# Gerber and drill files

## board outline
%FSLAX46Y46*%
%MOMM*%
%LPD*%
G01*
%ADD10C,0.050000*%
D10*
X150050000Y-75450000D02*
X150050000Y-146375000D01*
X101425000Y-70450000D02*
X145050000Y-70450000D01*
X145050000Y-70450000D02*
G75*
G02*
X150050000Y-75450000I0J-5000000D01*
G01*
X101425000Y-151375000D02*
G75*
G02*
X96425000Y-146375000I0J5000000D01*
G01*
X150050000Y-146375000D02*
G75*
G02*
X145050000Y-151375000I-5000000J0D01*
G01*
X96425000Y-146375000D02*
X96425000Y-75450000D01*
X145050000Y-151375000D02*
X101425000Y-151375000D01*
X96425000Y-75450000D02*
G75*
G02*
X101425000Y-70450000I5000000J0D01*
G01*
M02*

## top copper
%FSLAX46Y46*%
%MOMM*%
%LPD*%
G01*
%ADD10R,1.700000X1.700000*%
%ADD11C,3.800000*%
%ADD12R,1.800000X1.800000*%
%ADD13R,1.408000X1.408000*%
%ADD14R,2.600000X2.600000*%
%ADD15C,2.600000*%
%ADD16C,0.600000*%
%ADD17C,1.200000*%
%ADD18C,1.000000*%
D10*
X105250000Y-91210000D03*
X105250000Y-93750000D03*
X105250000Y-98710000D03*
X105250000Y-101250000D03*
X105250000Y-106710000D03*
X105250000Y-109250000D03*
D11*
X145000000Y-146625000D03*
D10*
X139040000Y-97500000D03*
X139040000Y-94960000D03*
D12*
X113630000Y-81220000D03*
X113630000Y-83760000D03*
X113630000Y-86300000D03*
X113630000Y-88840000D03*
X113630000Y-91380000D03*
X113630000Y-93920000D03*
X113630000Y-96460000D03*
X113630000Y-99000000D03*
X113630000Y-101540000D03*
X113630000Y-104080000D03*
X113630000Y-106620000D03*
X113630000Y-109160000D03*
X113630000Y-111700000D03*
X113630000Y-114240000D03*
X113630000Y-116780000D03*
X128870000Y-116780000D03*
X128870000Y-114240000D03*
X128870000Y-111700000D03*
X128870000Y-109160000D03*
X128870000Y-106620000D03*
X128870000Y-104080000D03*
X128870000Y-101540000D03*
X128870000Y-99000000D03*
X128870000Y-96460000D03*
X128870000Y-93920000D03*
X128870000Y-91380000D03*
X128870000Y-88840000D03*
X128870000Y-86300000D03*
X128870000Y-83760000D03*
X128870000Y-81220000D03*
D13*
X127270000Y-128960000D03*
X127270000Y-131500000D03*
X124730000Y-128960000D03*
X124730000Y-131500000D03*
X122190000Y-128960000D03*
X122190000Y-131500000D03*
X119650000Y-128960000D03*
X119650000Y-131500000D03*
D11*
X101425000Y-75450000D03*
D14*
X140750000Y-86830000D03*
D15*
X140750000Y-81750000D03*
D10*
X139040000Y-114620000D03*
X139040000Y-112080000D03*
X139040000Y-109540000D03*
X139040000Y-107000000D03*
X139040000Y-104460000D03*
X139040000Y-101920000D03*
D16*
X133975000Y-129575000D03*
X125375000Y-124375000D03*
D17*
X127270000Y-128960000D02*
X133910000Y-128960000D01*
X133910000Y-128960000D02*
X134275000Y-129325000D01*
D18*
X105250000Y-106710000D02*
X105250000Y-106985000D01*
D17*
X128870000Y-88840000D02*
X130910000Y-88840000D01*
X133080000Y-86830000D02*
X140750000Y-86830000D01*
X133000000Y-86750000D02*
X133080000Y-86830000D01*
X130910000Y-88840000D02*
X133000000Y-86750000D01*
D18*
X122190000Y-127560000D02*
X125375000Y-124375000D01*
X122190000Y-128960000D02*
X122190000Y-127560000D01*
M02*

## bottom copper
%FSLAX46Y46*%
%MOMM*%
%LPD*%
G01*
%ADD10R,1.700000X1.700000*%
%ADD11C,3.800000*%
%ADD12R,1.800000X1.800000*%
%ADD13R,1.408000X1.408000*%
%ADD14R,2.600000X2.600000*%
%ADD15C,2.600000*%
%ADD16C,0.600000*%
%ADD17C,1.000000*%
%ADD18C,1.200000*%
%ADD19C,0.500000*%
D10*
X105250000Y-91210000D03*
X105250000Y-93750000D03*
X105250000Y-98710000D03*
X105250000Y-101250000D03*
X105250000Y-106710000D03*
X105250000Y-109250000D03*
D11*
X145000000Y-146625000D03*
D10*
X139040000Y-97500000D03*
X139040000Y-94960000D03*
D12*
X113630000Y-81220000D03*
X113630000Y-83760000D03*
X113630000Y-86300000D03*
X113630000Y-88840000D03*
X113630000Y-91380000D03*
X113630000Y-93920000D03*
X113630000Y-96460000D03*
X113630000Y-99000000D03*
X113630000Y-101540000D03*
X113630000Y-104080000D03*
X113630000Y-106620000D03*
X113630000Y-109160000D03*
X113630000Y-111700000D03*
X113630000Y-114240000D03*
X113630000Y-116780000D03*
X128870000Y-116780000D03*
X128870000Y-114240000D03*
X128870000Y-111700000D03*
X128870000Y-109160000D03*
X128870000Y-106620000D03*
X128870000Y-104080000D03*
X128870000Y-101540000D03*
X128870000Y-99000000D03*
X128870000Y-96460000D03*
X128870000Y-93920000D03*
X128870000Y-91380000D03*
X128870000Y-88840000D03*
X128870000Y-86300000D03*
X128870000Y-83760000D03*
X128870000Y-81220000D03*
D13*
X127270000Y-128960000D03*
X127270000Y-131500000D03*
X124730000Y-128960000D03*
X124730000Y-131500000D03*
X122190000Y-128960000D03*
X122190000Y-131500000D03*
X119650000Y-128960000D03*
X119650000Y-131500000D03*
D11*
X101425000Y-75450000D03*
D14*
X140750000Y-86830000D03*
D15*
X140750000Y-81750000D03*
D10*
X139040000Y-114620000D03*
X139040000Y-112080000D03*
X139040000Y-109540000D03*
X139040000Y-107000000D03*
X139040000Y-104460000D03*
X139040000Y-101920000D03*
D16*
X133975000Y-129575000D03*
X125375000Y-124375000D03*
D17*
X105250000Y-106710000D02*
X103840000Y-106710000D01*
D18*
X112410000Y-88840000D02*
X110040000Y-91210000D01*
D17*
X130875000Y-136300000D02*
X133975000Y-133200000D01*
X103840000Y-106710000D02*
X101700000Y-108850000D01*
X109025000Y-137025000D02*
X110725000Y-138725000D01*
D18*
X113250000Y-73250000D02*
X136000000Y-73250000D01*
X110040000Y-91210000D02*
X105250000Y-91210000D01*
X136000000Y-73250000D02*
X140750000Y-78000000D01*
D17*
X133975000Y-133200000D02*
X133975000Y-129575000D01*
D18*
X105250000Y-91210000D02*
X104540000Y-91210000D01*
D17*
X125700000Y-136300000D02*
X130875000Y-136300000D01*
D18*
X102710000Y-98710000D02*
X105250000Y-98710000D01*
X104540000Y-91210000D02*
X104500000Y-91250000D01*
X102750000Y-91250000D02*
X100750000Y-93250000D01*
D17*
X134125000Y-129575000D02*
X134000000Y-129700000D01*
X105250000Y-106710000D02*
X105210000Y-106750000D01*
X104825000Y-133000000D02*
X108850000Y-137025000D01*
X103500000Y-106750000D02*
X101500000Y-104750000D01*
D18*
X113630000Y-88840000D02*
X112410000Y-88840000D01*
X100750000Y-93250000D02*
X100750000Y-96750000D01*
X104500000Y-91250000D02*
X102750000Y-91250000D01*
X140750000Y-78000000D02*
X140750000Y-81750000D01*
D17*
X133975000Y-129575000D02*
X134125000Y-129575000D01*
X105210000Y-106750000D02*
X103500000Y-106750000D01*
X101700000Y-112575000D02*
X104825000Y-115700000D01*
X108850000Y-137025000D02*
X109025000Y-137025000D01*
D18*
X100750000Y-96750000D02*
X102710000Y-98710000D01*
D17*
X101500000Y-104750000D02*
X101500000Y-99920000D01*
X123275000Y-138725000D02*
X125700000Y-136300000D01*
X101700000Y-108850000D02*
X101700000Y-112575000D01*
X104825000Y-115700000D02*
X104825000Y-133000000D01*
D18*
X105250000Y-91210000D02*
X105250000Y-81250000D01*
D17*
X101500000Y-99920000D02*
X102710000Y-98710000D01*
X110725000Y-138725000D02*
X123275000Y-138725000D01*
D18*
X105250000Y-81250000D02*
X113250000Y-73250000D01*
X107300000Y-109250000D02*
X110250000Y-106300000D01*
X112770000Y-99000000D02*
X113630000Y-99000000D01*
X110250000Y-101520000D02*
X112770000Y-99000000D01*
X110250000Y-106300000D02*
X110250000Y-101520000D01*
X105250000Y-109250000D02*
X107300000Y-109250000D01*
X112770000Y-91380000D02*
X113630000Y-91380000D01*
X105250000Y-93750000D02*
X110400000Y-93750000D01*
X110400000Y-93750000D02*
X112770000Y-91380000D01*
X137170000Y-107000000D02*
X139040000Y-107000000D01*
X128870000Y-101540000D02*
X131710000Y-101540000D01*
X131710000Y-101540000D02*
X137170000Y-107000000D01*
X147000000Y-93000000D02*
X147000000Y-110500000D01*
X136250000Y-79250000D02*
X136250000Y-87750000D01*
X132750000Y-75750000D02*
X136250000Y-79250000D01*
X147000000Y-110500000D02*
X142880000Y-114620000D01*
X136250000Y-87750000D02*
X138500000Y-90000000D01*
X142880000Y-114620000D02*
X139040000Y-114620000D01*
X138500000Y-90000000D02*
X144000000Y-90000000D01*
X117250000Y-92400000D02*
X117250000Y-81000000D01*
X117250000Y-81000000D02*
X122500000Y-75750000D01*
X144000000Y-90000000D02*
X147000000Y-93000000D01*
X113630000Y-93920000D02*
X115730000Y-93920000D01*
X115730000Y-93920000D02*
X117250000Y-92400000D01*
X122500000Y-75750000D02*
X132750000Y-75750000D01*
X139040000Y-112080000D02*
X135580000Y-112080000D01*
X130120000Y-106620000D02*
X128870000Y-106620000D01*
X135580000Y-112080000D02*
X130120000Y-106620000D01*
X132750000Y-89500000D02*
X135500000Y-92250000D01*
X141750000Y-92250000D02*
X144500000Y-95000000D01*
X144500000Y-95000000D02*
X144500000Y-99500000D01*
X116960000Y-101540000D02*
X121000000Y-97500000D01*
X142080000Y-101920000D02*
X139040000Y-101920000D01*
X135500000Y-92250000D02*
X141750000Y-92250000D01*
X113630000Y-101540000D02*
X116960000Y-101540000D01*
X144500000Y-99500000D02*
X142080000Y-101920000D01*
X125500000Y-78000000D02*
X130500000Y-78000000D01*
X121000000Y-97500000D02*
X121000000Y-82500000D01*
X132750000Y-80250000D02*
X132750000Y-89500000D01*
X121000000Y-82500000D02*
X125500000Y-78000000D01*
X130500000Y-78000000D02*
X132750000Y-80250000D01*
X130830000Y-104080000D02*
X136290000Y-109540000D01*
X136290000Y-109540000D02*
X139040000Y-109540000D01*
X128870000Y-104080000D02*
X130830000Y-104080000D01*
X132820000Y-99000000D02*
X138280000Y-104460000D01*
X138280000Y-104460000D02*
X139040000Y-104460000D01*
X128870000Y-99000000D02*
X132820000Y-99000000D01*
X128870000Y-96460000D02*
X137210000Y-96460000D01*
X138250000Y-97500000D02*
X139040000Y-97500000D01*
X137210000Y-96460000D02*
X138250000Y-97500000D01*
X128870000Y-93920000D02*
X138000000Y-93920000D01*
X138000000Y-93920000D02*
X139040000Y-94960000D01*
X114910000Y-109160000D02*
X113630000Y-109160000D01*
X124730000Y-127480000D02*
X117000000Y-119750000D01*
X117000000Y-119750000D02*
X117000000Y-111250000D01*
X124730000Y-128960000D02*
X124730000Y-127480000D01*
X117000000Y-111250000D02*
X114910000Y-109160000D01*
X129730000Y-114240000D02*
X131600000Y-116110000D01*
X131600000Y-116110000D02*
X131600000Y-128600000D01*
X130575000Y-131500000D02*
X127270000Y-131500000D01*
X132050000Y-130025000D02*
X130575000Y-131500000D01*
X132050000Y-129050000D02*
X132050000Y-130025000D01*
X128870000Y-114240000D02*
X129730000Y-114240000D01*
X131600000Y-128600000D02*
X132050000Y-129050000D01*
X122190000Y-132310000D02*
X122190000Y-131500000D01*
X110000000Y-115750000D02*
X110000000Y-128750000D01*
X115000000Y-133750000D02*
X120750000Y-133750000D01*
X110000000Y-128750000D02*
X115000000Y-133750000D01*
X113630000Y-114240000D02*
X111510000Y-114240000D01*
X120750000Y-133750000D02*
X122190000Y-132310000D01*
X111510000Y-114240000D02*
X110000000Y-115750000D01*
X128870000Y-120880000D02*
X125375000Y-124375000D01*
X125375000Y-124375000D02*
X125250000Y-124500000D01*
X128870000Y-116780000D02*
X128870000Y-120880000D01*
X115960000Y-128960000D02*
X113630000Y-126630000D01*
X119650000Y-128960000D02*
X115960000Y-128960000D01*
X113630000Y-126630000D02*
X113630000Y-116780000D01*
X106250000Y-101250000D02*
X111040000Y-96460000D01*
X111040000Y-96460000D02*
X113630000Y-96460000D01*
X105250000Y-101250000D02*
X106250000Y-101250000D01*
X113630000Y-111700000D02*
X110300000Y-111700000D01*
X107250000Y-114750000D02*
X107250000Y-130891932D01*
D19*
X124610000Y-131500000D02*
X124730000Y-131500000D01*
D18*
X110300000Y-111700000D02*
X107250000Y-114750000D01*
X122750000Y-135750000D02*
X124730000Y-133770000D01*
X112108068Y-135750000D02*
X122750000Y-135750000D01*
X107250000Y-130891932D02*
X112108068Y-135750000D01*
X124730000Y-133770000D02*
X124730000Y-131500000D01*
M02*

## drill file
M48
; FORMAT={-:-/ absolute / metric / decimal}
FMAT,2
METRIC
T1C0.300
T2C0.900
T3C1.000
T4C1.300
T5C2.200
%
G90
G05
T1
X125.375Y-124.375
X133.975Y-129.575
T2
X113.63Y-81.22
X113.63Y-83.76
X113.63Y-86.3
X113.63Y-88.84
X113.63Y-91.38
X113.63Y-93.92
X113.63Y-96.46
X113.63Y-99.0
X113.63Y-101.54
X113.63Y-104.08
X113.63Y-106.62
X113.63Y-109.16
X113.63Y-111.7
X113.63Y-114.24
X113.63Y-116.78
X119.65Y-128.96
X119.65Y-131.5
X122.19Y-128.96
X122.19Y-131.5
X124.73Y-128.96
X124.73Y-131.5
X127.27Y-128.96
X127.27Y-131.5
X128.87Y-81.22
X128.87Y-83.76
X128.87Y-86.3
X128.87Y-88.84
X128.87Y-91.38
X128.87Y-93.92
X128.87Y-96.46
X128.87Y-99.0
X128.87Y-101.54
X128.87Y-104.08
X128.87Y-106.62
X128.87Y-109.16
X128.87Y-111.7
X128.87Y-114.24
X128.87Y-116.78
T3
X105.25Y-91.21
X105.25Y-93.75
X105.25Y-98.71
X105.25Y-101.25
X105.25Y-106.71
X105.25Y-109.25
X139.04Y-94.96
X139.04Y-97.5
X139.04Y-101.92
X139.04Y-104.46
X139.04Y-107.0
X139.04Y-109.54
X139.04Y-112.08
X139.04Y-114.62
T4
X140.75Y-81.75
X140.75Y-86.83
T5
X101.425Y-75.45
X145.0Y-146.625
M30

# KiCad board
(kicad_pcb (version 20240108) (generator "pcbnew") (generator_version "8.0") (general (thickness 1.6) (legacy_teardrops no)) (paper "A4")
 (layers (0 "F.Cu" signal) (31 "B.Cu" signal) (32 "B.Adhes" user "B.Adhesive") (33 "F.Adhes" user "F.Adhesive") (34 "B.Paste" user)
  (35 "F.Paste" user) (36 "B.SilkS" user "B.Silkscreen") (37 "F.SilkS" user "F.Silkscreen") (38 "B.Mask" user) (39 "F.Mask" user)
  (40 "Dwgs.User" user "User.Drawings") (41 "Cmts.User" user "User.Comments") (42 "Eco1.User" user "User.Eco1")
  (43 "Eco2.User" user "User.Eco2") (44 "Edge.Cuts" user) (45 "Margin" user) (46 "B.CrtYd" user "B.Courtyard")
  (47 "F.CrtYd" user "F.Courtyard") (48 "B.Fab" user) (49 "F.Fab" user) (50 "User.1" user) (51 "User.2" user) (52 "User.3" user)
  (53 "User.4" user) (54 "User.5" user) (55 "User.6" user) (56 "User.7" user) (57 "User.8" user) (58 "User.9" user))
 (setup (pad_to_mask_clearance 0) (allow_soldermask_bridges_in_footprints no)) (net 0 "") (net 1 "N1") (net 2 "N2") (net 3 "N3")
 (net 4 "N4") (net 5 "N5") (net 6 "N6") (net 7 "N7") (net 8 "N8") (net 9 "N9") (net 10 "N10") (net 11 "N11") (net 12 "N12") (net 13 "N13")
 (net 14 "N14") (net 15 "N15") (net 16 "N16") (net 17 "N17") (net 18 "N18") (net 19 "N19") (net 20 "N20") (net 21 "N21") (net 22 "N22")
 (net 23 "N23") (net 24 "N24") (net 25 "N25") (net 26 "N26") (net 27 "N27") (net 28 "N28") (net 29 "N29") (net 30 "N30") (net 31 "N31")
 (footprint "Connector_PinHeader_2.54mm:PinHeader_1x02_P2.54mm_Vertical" (layer "F.Cu") (at 105.25 91.21)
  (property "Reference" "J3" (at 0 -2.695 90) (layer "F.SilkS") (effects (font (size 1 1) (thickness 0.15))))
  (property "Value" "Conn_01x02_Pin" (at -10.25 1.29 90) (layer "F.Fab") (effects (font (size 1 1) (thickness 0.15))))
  (pad "1" thru_hole rect (at 0 0) (size 1.7 1.7) (drill 1) (layers "*.Cu" "*.Mask") (remove_unused_layers no) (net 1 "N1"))
  (pad "2" thru_hole rect (at 0 2.54) (size 1.7 1.7) (drill 1) (layers "*.Cu" "*.Mask") (remove_unused_layers no) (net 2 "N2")))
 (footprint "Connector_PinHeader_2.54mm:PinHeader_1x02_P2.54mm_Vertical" (layer "F.Cu") (at 105.25 98.71)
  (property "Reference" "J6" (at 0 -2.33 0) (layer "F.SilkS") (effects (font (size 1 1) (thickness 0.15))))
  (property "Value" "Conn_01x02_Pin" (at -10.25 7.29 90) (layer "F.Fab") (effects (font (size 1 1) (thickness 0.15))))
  (pad "1" thru_hole rect (at 0 0) (size 1.7 1.7) (drill 1) (layers "*.Cu" "*.Mask") (remove_unused_layers no) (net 1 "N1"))
  (pad "2" thru_hole rect (at 0 2.54) (size 1.7 1.7) (drill 1) (layers "*.Cu" "*.Mask") (remove_unused_layers no) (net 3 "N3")))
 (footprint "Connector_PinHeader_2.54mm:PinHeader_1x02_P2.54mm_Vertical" (layer "F.Cu") (at 105.25 106.71)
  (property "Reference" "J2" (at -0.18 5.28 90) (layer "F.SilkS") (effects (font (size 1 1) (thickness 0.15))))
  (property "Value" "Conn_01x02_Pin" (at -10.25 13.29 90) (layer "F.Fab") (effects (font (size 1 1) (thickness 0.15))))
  (pad "1" thru_hole rect (at 0 0) (size 1.7 1.7) (drill 1) (layers "*.Cu" "*.Mask") (remove_unused_layers no) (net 1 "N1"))
  (pad "2" thru_hole rect (at 0 2.54) (size 1.7 1.7) (drill 1) (layers "*.Cu" "*.Mask") (remove_unused_layers no) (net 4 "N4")))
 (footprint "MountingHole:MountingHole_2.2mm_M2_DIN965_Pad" (layer "F.Cu") (at 145 146.625)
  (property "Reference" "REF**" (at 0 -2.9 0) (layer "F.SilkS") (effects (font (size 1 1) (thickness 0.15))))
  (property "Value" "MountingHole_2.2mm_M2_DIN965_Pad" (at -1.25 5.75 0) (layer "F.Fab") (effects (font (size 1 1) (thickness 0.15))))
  (pad "2" thru_hole circle (at 0 0) (size 3.8 3.8) (drill 2.2) (layers "*.Cu" "*.Mask") (remove_unused_layers no)))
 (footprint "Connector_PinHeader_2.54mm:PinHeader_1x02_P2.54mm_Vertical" (layer "F.Cu") (at 139.04 97.5 180)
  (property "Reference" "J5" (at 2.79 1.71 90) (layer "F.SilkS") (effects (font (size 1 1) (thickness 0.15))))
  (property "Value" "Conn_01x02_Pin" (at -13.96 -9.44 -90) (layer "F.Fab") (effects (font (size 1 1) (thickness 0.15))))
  (pad "1" thru_hole rect (at 0 0 180) (size 1.7 1.7) (drill 1) (layers "*.Cu" "*.Mask") (remove_unused_layers no) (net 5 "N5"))
  (pad "2" thru_hole rect (at 0 2.54 180) (size 1.7 1.7) (drill 1) (layers "*.Cu" "*.Mask") (remove_unused_layers no) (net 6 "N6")))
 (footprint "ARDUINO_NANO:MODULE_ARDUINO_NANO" (layer "F.Cu") (at 121.25 99)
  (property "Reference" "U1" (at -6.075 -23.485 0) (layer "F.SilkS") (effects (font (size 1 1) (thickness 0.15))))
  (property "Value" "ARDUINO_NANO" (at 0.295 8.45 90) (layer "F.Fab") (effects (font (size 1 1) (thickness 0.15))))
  (pad "1" thru_hole rect (at -7.62 -17.78) (size 1.8 1.8) (drill 0.9) (layers "*.Cu" "*.Mask") (remove_unused_layers no) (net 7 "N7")
   (solder_mask_margin 0.102))
  (pad "2" thru_hole rect (at -7.62 -15.24) (size 1.8 1.8) (drill 0.9) (layers "*.Cu" "*.Mask") (remove_unused_layers no) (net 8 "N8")
   (solder_mask_margin 0.102))
  (pad "3" thru_hole rect (at -7.62 -12.7) (size 1.8 1.8) (drill 0.9) (layers "*.Cu" "*.Mask") (remove_unused_layers no) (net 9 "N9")
   (solder_mask_margin 0.102))
  (pad "4" thru_hole rect (at -7.62 -10.16) (size 1.8 1.8) (drill 0.9) (layers "*.Cu" "*.Mask") (remove_unused_layers no) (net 1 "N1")
   (solder_mask_margin 0.102))
  (pad "5" thru_hole rect (at -7.62 -7.62) (size 1.8 1.8) (drill 0.9) (layers "*.Cu" "*.Mask") (remove_unused_layers no) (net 2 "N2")
   (solder_mask_margin 0.102))
  (pad "6" thru_hole rect (at -7.62 -5.08) (size 1.8 1.8) (drill 0.9) (layers "*.Cu" "*.Mask") (remove_unused_layers no) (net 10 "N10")
   (solder_mask_margin 0.102))
  (pad "7" thru_hole rect (at -7.62 -2.54) (size 1.8 1.8) (drill 0.9) (layers "*.Cu" "*.Mask") (remove_unused_layers no) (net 3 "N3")
   (solder_mask_margin 0.102))
  (pad "8" thru_hole rect (at -7.62 0) (size 1.8 1.8) (drill 0.9) (layers "*.Cu" "*.Mask") (remove_unused_layers no) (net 4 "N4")
   (solder_mask_margin 0.102))
  (pad "9" thru_hole rect (at -7.62 2.54) (size 1.8 1.8) (drill 0.9) (layers "*.Cu" "*.Mask") (remove_unused_layers no) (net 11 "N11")
   (solder_mask_margin 0.102))
  (pad "10" thru_hole rect (at -7.62 5.08) (size 1.8 1.8) (drill 0.9) (layers "*.Cu" "*.Mask") (remove_unused_layers no) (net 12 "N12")
   (solder_mask_margin 0.102))
  (pad "11" thru_hole rect (at -7.62 7.62) (size 1.8 1.8) (drill 0.9) (layers "*.Cu" "*.Mask") (remove_unused_layers no) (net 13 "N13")
   (solder_mask_margin 0.102))
  (pad "12" thru_hole rect (at -7.62 10.16) (size 1.8 1.8) (drill 0.9) (layers "*.Cu" "*.Mask") (remove_unused_layers no) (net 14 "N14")
   (solder_mask_margin 0.102))
  (pad "13" thru_hole rect (at -7.62 12.7) (size 1.8 1.8) (drill 0.9) (layers "*.Cu" "*.Mask") (remove_unused_layers no) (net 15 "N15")
   (solder_mask_margin 0.102))
  (pad "14" thru_hole rect (at -7.62 15.24) (size 1.8 1.8) (drill 0.9) (layers "*.Cu" "*.Mask") (remove_unused_layers no) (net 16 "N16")
   (solder_mask_margin 0.102))
  (pad "15" thru_hole rect (at -7.62 17.78) (size 1.8 1.8) (drill 0.9) (layers "*.Cu" "*.Mask") (remove_unused_layers no) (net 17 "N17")
   (solder_mask_margin 0.102))
  (pad "16" thru_hole rect (at 7.62 17.78) (size 1.8 1.8) (drill 0.9) (layers "*.Cu" "*.Mask") (remove_unused_layers no) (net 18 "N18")
   (solder_mask_margin 0.102))
  (pad "17" thru_hole rect (at 7.62 15.24) (size 1.8 1.8) (drill 0.9) (layers "*.Cu" "*.Mask") (remove_unused_layers no) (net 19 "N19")
   (solder_mask_margin 0.102))
  (pad "18" thru_hole rect (at 7.62 12.7) (size 1.8 1.8) (drill 0.9) (layers "*.Cu" "*.Mask") (remove_unused_layers no) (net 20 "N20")
   (solder_mask_margin 0.102))
  (pad "19" thru_hole rect (at 7.62 10.16) (size 1.8 1.8) (drill 0.9) (layers "*.Cu" "*.Mask") (remove_unused_layers no) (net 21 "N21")
   (solder_mask_margin 0.102))
  (pad "20" thru_hole rect (at 7.62 7.62) (size 1.8 1.8) (drill 0.9) (layers "*.Cu" "*.Mask") (remove_unused_layers no) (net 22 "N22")
   (solder_mask_margin 0.102))
  (pad "21" thru_hole rect (at 7.62 5.08) (size 1.8 1.8) (drill 0.9) (layers "*.Cu" "*.Mask") (remove_unused_layers no) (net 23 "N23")
   (solder_mask_margin 0.102))
  (pad "22" thru_hole rect (at 7.62 2.54) (size 1.8 1.8) (drill 0.9) (layers "*.Cu" "*.Mask") (remove_unused_layers no) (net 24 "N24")
   (solder_mask_margin 0.102))
  (pad "23" thru_hole rect (at 7.62 0) (size 1.8 1.8) (drill 0.9) (layers "*.Cu" "*.Mask") (remove_unused_layers no) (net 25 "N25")
   (solder_mask_margin 0.102))
  (pad "24" thru_hole rect (at 7.62 -2.54) (size 1.8 1.8) (drill 0.9) (layers "*.Cu" "*.Mask") (remove_unused_layers no) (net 5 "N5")
   (solder_mask_margin 0.102))
  (pad "25" thru_hole rect (at 7.62 -5.08) (size 1.8 1.8) (drill 0.9) (layers "*.Cu" "*.Mask") (remove_unused_layers no) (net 6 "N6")
   (solder_mask_margin 0.102))
  (pad "26" thru_hole rect (at 7.62 -7.62) (size 1.8 1.8) (drill 0.9) (layers "*.Cu" "*.Mask") (remove_unused_layers no) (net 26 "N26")
   (solder_mask_margin 0.102))
  (pad "27" thru_hole rect (at 7.62 -10.16) (size 1.8 1.8) (drill 0.9) (layers "*.Cu" "*.Mask") (remove_unused_layers no) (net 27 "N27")
   (solder_mask_margin 0.102))
  (pad "28" thru_hole rect (at 7.62 -12.7) (size 1.8 1.8) (drill 0.9) (layers "*.Cu" "*.Mask") (remove_unused_layers no) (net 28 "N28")
   (solder_mask_margin 0.102))
  (pad "29" thru_hole rect (at 7.62 -15.24) (size 1.8 1.8) (drill 0.9) (layers "*.Cu" "*.Mask") (remove_unused_layers no) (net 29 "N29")
   (solder_mask_margin 0.102))
  (pad "30" thru_hole rect (at 7.62 -17.78) (size 1.8 1.8) (drill 0.9) (layers "*.Cu" "*.Mask") (remove_unused_layers no) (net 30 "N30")
   (solder_mask_margin 0.102)))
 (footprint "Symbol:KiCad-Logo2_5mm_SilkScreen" (layer "F.Cu") (at 142.2 131.375 90)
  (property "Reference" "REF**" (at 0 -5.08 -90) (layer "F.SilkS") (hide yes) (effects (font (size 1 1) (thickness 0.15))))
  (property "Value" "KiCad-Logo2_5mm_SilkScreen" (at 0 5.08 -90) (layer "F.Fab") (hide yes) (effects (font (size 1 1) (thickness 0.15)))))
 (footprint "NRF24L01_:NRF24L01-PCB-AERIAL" (layer "F.Cu") (at 123.46 130.23 180)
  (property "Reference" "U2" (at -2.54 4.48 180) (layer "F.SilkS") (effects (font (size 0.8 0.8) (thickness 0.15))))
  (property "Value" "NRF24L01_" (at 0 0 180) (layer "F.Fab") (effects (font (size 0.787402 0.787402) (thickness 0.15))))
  (pad "P$1" thru_hole rect (at -3.81 1.27 180) (size 1.408 1.408) (drill 0.9) (layers "*.Cu" "*.Mask") (remove_unused_layers no)
   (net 1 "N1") (solder_mask_margin 0.102))
  (pad "P$2" thru_hole rect (at -3.81 -1.27 180) (size 1.408 1.408) (drill 0.9) (layers "*.Cu" "*.Mask") (remove_unused_layers no)
   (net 19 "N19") (solder_mask_margin 0.102))
  (pad "P$3" thru_hole rect (at -1.27 1.27 180) (size 1.408 1.408) (drill 0.9) (layers "*.Cu" "*.Mask") (remove_unused_layers no)
   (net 14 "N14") (solder_mask_margin 0.102))
  (pad "P$4" thru_hole rect (at -1.27 -1.27 180) (size 1.408 1.408) (drill 0.9) (layers "*.Cu" "*.Mask") (remove_unused_layers no)
   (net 15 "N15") (solder_mask_margin 0.102))
  (pad "P$5" thru_hole rect (at 1.27 1.27 180) (size 1.408 1.408) (drill 0.9) (layers "*.Cu" "*.Mask") (remove_unused_layers no)
   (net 18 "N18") (solder_mask_margin 0.102))
  (pad "P$6" thru_hole rect (at 1.27 -1.27 180) (size 1.408 1.408) (drill 0.9) (layers "*.Cu" "*.Mask") (remove_unused_layers no)
   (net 16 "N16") (solder_mask_margin 0.102))
  (pad "P$7" thru_hole rect (at 3.81 1.27 180) (size 1.408 1.408) (drill 0.9) (layers "*.Cu" "*.Mask") (remove_unused_layers no)
   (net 17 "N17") (solder_mask_margin 0.102))
  (pad "P$8" thru_hole rect (at 3.81 -1.27 180) (size 1.408 1.408) (drill 0.9) (layers "*.Cu" "*.Mask") (remove_unused_layers no)
   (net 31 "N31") (solder_mask_margin 0.102)))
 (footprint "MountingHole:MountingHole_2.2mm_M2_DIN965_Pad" (layer "F.Cu") (at 101.425 75.45)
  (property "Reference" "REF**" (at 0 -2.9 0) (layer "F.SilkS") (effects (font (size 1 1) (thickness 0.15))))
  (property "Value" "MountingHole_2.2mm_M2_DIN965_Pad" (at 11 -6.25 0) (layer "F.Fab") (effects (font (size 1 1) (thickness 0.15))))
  (pad "1" thru_hole circle (at 0 0) (size 3.8 3.8) (drill 2.2) (layers "*.Cu" "*.Mask") (remove_unused_layers no)))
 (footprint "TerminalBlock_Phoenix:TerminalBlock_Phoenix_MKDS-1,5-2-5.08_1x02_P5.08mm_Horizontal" (layer "F.Cu") (at 140.75 86.83 90)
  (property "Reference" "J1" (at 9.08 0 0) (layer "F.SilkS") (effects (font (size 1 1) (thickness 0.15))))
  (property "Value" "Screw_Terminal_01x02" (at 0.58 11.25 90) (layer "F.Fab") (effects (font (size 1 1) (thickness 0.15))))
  (pad "1" thru_hole rect (at 0 0 90) (size 2.6 2.6) (drill 1.3) (layers "*.Cu" "*.Mask") (remove_unused_layers no) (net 27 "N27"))
  (pad "2" thru_hole circle (at 5.08 0 90) (size 2.6 2.6) (drill 1.3) (layers "*.Cu" "*.Mask") (remove_unused_layers no) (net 1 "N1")))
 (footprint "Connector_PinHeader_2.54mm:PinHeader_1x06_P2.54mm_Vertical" (layer "F.Cu") (at 139.04 114.62 180)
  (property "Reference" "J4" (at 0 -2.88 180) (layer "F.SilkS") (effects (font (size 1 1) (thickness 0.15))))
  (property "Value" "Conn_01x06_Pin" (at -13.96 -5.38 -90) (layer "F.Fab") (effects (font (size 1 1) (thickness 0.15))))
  (pad "1" thru_hole rect (at 0 0 180) (size 1.7 1.7) (drill 1) (layers "*.Cu" "*.Mask") (remove_unused_layers no) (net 10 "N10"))
  (pad "2" thru_hole rect (at 0 2.54 180) (size 1.7 1.7) (drill 1) (layers "*.Cu" "*.Mask") (remove_unused_layers no) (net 22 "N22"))
  (pad "3" thru_hole rect (at 0 5.08 180) (size 1.7 1.7) (drill 1) (layers "*.Cu" "*.Mask") (remove_unused_layers no) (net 23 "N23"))
  (pad "4" thru_hole rect (at 0 7.62 180) (size 1.7 1.7) (drill 1) (layers "*.Cu" "*.Mask") (remove_unused_layers no) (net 24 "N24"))
  (pad "5" thru_hole rect (at 0 10.16 180) (size 1.7 1.7) (drill 1) (layers "*.Cu" "*.Mask") (remove_unused_layers no) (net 25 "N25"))
  (pad "6" thru_hole rect (at 0 12.7 180) (size 1.7 1.7) (drill 1) (layers "*.Cu" "*.Mask") (remove_unused_layers no) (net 11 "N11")))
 (gr_line (start 150.05 75.45) (end 150.05 146.375) (stroke (width 0.05) (type default)) (layer "Edge.Cuts"))
 (gr_line (start 101.425 70.45) (end 145.05 70.45) (stroke (width 0.05) (type default)) (layer "Edge.Cuts"))
 (gr_arc (start 145.05 70.45) (mid 148.585534 71.914466) (end 150.05 75.45) (stroke (width 0.05) (type default)) (layer "Edge.Cuts"))
 (gr_arc (start 101.425 151.375) (mid 97.889466 149.910534) (end 96.425 146.375) (stroke (width 0.05) (type default)) (layer "Edge.Cuts"))
 (gr_arc (start 150.05 146.375) (mid 148.585534 149.910534) (end 145.05 151.375) (stroke (width 0.05) (type default)) (layer "Edge.Cuts"))
 (gr_line (start 96.425 146.375) (end 96.425 75.45) (stroke (width 0.05) (type default)) (layer "Edge.Cuts"))
 (gr_line (start 145.05 151.375) (end 101.425 151.375) (stroke (width 0.05) (type default)) (layer "Edge.Cuts"))
 (gr_arc (start 96.425 75.45) (mid 97.889466 71.914466) (end 101.425 70.45) (stroke (width 0.05) (type default)) (layer "Edge.Cuts"))
 (segment (start 127.27 128.96) (end 133.91 128.96) (width 1.2) (layer "F.Cu") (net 1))
 (segment (start 133.91 128.96) (end 134.275 129.325) (width 1.2) (layer "F.Cu") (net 1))
 (segment (start 105.25 106.71) (end 105.25 106.985) (width 1) (layer "F.Cu") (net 1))
 (via (at 133.975 129.575) (size 0.6) (drill 0.3) (layers "F.Cu" "B.Cu") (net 1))
 (segment (start 105.25 106.71) (end 103.84 106.71) (width 1) (layer "B.Cu") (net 1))
 (segment (start 112.41 88.84) (end 110.04 91.21) (width 1.2) (layer "B.Cu") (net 1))
 (segment (start 130.875 136.3) (end 133.975 133.2) (width 1) (layer "B.Cu") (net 1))
 (segment (start 103.84 106.71) (end 101.7 108.85) (width 1) (layer "B.Cu") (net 1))
 (segment (start 109.025 137.025) (end 110.725 138.725) (width 1) (layer "B.Cu") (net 1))
 (segment (start 113.25 73.25) (end 136 73.25) (width 1.2) (layer "B.Cu") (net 1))
 (segment (start 110.04 91.21) (end 105.25 91.21) (width 1.2) (layer "B.Cu") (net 1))
 (segment (start 136 73.25) (end 140.75 78) (width 1.2) (layer "B.Cu") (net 1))
 (segment (start 133.975 133.2) (end 133.975 129.575) (width 1) (layer "B.Cu") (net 1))
 (segment (start 105.25 91.21) (end 104.54 91.21) (width 1.2) (layer "B.Cu") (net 1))
 (segment (start 125.7 136.3) (end 130.875 136.3) (width 1) (layer "B.Cu") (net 1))
 (segment (start 102.71 98.71) (end 105.25 98.71) (width 1.2) (layer "B.Cu") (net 1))
 (segment (start 104.54 91.21) (end 104.5 91.25) (width 1.2) (layer "B.Cu") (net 1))
 (segment (start 102.75 91.25) (end 100.75 93.25) (width 1.2) (layer "B.Cu") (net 1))
 (segment (start 134.125 129.575) (end 134 129.7) (width 1) (layer "B.Cu") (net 1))
 (segment (start 105.25 106.71) (end 105.21 106.75) (width 1) (layer "B.Cu") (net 1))
 (segment (start 104.825 133) (end 108.85 137.025) (width 1) (layer "B.Cu") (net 1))
 (segment (start 103.5 106.75) (end 101.5 104.75) (width 1) (layer "B.Cu") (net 1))
 (segment (start 113.63 88.84) (end 112.41 88.84) (width 1.2) (layer "B.Cu") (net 1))
 (segment (start 100.75 93.25) (end 100.75 96.75) (width 1.2) (layer "B.Cu") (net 1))
 (segment (start 104.5 91.25) (end 102.75 91.25) (width 1.2) (layer "B.Cu") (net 1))
 (segment (start 140.75 78) (end 140.75 81.75) (width 1.2) (layer "B.Cu") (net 1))
 (segment (start 133.975 129.575) (end 134.125 129.575) (width 1) (layer "B.Cu") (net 1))
 (segment (start 105.21 106.75) (end 103.5 106.75) (width 1) (layer "B.Cu") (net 1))
 (segment (start 101.7 112.575) (end 104.825 115.7) (width 1) (layer "B.Cu") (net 1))
 (segment (start 108.85 137.025) (end 109.025 137.025) (width 1) (layer "B.Cu") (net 1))
 (segment (start 100.75 96.75) (end 102.71 98.71) (width 1.2) (layer "B.Cu") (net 1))
 (segment (start 101.5 104.75) (end 101.5 99.92) (width 1) (layer "B.Cu") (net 1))
 (segment (start 123.275 138.725) (end 125.7 136.3) (width 1) (layer "B.Cu") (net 1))
 (segment (start 101.7 108.85) (end 101.7 112.575) (width 1) (layer "B.Cu") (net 1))
 (segment (start 104.825 115.7) (end 104.825 133) (width 1) (layer "B.Cu") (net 1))
 (segment (start 105.25 91.21) (end 105.25 81.25) (width 1.2) (layer "B.Cu") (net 1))
 (segment (start 101.5 99.92) (end 102.71 98.71) (width 1) (layer "B.Cu") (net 1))
 (segment (start 110.725 138.725) (end 123.275 138.725) (width 1) (layer "B.Cu") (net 1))
 (segment (start 105.25 81.25) (end 113.25 73.25) (width 1.2) (layer "B.Cu") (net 1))
 (segment (start 128.87 88.84) (end 130.91 88.84) (width 1.2) (layer "F.Cu") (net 27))
 (segment (start 133.08 86.83) (end 140.75 86.83) (width 1.2) (layer "F.Cu") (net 27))
 (segment (start 133 86.75) (end 133.08 86.83) (width 1.2) (layer "F.Cu") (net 27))
 (segment (start 130.91 88.84) (end 133 86.75) (width 1.2) (layer "F.Cu") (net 27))
 (segment (start 107.3 109.25) (end 110.25 106.3) (width 1.2) (layer "B.Cu") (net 4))
 (segment (start 112.77 99) (end 113.63 99) (width 1.2) (layer "B.Cu") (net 4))
 (segment (start 110.25 101.52) (end 112.77 99) (width 1.2) (layer "B.Cu") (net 4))
 (segment (start 110.25 106.3) (end 110.25 101.52) (width 1.2) (layer "B.Cu") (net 4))
 (segment (start 105.25 109.25) (end 107.3 109.25) (width 1.2) (layer "B.Cu") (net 4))
 (segment (start 112.77 91.38) (end 113.63 91.38) (width 1.2) (layer "B.Cu") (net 2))
 (segment (start 105.25 93.75) (end 110.4 93.75) (width 1.2) (layer "B.Cu") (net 2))
 (segment (start 110.4 93.75) (end 112.77 91.38) (width 1.2) (layer "B.Cu") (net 2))
 (segment (start 137.17 107) (end 139.04 107) (width 1.2) (layer "B.Cu") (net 24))
 (segment (start 128.87 101.54) (end 131.71 101.54) (width 1.2) (layer "B.Cu") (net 24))
 (segment (start 131.71 101.54) (end 137.17 107) (width 1.2) (layer "B.Cu") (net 24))
 (segment (start 147 93) (end 147 110.5) (width 1.2) (layer "B.Cu") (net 10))
 (segment (start 136.25 79.25) (end 136.25 87.75) (width 1.2) (layer "B.Cu") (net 10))
 (segment (start 132.75 75.75) (end 136.25 79.25) (width 1.2) (layer "B.Cu") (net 10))
 (segment (start 147 110.5) (end 142.88 114.62) (width 1.2) (layer "B.Cu") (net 10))
 (segment (start 136.25 87.75) (end 138.5 90) (width 1.2) (layer "B.Cu") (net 10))
 (segment (start 142.88 114.62) (end 139.04 114.62) (width 1.2) (layer "B.Cu") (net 10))
 (segment (start 138.5 90) (end 144 90) (width 1.2) (layer "B.Cu") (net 10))
 (segment (start 117.25 92.4) (end 117.25 81) (width 1.2) (layer "B.Cu") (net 10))
 (segment (start 117.25 81) (end 122.5 75.75) (width 1.2) (layer "B.Cu") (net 10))
 (segment (start 144 90) (end 147 93) (width 1.2) (layer "B.Cu") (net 10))
 (segment (start 113.63 93.92) (end 115.73 93.92) (width 1.2) (layer "B.Cu") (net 10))
 (segment (start 115.73 93.92) (end 117.25 92.4) (width 1.2) (layer "B.Cu") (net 10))
 (segment (start 122.5 75.75) (end 132.75 75.75) (width 1.2) (layer "B.Cu") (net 10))
 (segment (start 139.04 112.08) (end 135.58 112.08) (width 1.2) (layer "B.Cu") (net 22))
 (segment (start 130.12 106.62) (end 128.87 106.62) (width 1.2) (layer "B.Cu") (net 22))
 (segment (start 135.58 112.08) (end 130.12 106.62) (width 1.2) (layer "B.Cu") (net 22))
 (segment (start 132.75 89.5) (end 135.5 92.25) (width 1.2) (layer "B.Cu") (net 11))
 (segment (start 141.75 92.25) (end 144.5 95) (width 1.2) (layer "B.Cu") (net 11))
 (segment (start 144.5 95) (end 144.5 99.5) (width 1.2) (layer "B.Cu") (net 11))
 (segment (start 116.96 101.54) (end 121 97.5) (width 1.2) (layer "B.Cu") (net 11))
 (segment (start 142.08 101.92) (end 139.04 101.92) (width 1.2) (layer "B.Cu") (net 11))
 (segment (start 135.5 92.25) (end 141.75 92.25) (width 1.2) (layer "B.Cu") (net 11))
 (segment (start 113.63 101.54) (end 116.96 101.54) (width 1.2) (layer "B.Cu") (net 11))
 (segment (start 144.5 99.5) (end 142.08 101.92) (width 1.2) (layer "B.Cu") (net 11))
 (segment (start 125.5 78) (end 130.5 78) (width 1.2) (layer "B.Cu") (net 11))
 (segment (start 121 97.5) (end 121 82.5) (width 1.2) (layer "B.Cu") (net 11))
 (segment (start 132.75 80.25) (end 132.75 89.5) (width 1.2) (layer "B.Cu") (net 11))
 (segment (start 121 82.5) (end 125.5 78) (width 1.2) (layer "B.Cu") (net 11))
 (segment (start 130.5 78) (end 132.75 80.25) (width 1.2) (layer "B.Cu") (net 11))
 (segment (start 130.83 104.08) (end 136.29 109.54) (width 1.2) (layer "B.Cu") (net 23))
 (segment (start 136.29 109.54) (end 139.04 109.54) (width 1.2) (layer "B.Cu") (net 23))
 (segment (start 128.87 104.08) (end 130.83 104.08) (width 1.2) (layer "B.Cu") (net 23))
 (segment (start 132.82 99) (end 138.28 104.46) (width 1.2) (layer "B.Cu") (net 25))
 (segment (start 138.28 104.46) (end 139.04 104.46) (width 1.2) (layer "B.Cu") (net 25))
 (segment (start 128.87 99) (end 132.82 99) (width 1.2) (layer "B.Cu") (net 25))
 (segment (start 128.87 96.46) (end 137.21 96.46) (width 1.2) (layer "B.Cu") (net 5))
 (segment (start 138.25 97.5) (end 139.04 97.5) (width 1.2) (layer "B.Cu") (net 5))
 (segment (start 137.21 96.46) (end 138.25 97.5) (width 1.2) (layer "B.Cu") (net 5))
 (segment (start 128.87 93.92) (end 138 93.92) (width 1.2) (layer "B.Cu") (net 6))
 (segment (start 138 93.92) (end 139.04 94.96) (width 1.2) (layer "B.Cu") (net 6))
 (segment (start 114.91 109.16) (end 113.63 109.16) (width 1.2) (layer "B.Cu") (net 14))
 (segment (start 124.73 127.48) (end 117 119.75) (width 1.2) (layer "B.Cu") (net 14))
 (segment (start 117 119.75) (end 117 111.25) (width 1.2) (layer "B.Cu") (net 14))
 (segment (start 124.73 128.96) (end 124.73 127.48) (width 1.2) (layer "B.Cu") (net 14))
 (segment (start 117 111.25) (end 114.91 109.16) (width 1.2) (layer "B.Cu") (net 14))
 (segment (start 129.73 114.24) (end 131.6 116.11) (width 1.2) (layer "B.Cu") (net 19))
 (segment (start 131.6 116.11) (end 131.6 128.6) (width 1.2) (layer "B.Cu") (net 19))
 (segment (start 130.575 131.5) (end 127.27 131.5) (width 1.2) (layer "B.Cu") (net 19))
 (segment (start 132.05 130.025) (end 130.575 131.5) (width 1.2) (layer "B.Cu") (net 19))
 (segment (start 132.05 129.05) (end 132.05 130.025) (width 1.2) (layer "B.Cu") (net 19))
 (segment (start 128.87 114.24) (end 129.73 114.24) (width 1.2) (layer "B.Cu") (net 19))
 (segment (start 131.6 128.6) (end 132.05 129.05) (width 1.2) (layer "B.Cu") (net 19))
 (segment (start 122.19 132.31) (end 122.19 131.5) (width 1.2) (layer "B.Cu") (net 16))
 (segment (start 110 115.75) (end 110 128.75) (width 1.2) (layer "B.Cu") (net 16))
 (segment (start 115 133.75) (end 120.75 133.75) (width 1.2) (layer "B.Cu") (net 16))
 (segment (start 110 128.75) (end 115 133.75) (width 1.2) (layer "B.Cu") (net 16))
 (segment (start 113.63 114.24) (end 111.51 114.24) (width 1.2) (layer "B.Cu") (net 16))
 (segment (start 120.75 133.75) (end 122.19 132.31) (width 1.2) (layer "B.Cu") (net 16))
 (segment (start 111.51 114.24) (end 110 115.75) (width 1.2) (layer "B.Cu") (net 16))
 (segment (start 122.19 127.56) (end 125.375 124.375) (width 1) (layer "F.Cu") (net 18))
 (segment (start 122.19 128.96) (end 122.19 127.56) (width 1) (layer "F.Cu") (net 18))
 (via (at 125.375 124.375) (size 0.6) (drill 0.3) (layers "F.Cu" "B.Cu") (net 18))
 (segment (start 128.87 120.88) (end 125.375 124.375) (width 1.2) (layer "B.Cu") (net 18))
 (segment (start 125.375 124.375) (end 125.25 124.5) (width 1.2) (layer "B.Cu") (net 18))
 (segment (start 128.87 116.78) (end 128.87 120.88) (width 1.2) (layer "B.Cu") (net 18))
 (segment (start 115.96 128.96) (end 113.63 126.63) (width 1.2) (layer "B.Cu") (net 17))
 (segment (start 119.65 128.96) (end 115.96 128.96) (width 1.2) (layer "B.Cu") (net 17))
 (segment (start 113.63 126.63) (end 113.63 116.78) (width 1.2) (layer "B.Cu") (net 17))
 (segment (start 106.25 101.25) (end 111.04 96.46) (width 1.2) (layer "B.Cu") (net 3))
 (segment (start 111.04 96.46) (end 113.63 96.46) (width 1.2) (layer "B.Cu") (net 3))
 (segment (start 105.25 101.25) (end 106.25 101.25) (width 1.2) (layer "B.Cu") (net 3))
 (segment (start 113.63 111.7) (end 110.3 111.7) (width 1.2) (layer "B.Cu") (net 15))
 (segment (start 107.25 114.75) (end 107.25 130.891932) (width 1.2) (layer "B.Cu") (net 15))
 (segment (start 124.61 131.5) (end 124.73 131.5) (width 0.5) (layer "B.Cu") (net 15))
 (segment (start 110.3 111.7) (end 107.25 114.75) (width 1.2) (layer "B.Cu") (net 15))
 (segment (start 122.75 135.75) (end 124.73 133.77) (width 1.2) (layer "B.Cu") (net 15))
 (segment (start 112.108068 135.75) (end 122.75 135.75) (width 1.2) (layer "B.Cu") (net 15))
 (segment (start 107.25 130.891932) (end 112.108068 135.75) (width 1.2) (layer "B.Cu") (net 15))
 (segment (start 124.73 133.77) (end 124.73 131.5) (width 1.2) (layer "B.Cu") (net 15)))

